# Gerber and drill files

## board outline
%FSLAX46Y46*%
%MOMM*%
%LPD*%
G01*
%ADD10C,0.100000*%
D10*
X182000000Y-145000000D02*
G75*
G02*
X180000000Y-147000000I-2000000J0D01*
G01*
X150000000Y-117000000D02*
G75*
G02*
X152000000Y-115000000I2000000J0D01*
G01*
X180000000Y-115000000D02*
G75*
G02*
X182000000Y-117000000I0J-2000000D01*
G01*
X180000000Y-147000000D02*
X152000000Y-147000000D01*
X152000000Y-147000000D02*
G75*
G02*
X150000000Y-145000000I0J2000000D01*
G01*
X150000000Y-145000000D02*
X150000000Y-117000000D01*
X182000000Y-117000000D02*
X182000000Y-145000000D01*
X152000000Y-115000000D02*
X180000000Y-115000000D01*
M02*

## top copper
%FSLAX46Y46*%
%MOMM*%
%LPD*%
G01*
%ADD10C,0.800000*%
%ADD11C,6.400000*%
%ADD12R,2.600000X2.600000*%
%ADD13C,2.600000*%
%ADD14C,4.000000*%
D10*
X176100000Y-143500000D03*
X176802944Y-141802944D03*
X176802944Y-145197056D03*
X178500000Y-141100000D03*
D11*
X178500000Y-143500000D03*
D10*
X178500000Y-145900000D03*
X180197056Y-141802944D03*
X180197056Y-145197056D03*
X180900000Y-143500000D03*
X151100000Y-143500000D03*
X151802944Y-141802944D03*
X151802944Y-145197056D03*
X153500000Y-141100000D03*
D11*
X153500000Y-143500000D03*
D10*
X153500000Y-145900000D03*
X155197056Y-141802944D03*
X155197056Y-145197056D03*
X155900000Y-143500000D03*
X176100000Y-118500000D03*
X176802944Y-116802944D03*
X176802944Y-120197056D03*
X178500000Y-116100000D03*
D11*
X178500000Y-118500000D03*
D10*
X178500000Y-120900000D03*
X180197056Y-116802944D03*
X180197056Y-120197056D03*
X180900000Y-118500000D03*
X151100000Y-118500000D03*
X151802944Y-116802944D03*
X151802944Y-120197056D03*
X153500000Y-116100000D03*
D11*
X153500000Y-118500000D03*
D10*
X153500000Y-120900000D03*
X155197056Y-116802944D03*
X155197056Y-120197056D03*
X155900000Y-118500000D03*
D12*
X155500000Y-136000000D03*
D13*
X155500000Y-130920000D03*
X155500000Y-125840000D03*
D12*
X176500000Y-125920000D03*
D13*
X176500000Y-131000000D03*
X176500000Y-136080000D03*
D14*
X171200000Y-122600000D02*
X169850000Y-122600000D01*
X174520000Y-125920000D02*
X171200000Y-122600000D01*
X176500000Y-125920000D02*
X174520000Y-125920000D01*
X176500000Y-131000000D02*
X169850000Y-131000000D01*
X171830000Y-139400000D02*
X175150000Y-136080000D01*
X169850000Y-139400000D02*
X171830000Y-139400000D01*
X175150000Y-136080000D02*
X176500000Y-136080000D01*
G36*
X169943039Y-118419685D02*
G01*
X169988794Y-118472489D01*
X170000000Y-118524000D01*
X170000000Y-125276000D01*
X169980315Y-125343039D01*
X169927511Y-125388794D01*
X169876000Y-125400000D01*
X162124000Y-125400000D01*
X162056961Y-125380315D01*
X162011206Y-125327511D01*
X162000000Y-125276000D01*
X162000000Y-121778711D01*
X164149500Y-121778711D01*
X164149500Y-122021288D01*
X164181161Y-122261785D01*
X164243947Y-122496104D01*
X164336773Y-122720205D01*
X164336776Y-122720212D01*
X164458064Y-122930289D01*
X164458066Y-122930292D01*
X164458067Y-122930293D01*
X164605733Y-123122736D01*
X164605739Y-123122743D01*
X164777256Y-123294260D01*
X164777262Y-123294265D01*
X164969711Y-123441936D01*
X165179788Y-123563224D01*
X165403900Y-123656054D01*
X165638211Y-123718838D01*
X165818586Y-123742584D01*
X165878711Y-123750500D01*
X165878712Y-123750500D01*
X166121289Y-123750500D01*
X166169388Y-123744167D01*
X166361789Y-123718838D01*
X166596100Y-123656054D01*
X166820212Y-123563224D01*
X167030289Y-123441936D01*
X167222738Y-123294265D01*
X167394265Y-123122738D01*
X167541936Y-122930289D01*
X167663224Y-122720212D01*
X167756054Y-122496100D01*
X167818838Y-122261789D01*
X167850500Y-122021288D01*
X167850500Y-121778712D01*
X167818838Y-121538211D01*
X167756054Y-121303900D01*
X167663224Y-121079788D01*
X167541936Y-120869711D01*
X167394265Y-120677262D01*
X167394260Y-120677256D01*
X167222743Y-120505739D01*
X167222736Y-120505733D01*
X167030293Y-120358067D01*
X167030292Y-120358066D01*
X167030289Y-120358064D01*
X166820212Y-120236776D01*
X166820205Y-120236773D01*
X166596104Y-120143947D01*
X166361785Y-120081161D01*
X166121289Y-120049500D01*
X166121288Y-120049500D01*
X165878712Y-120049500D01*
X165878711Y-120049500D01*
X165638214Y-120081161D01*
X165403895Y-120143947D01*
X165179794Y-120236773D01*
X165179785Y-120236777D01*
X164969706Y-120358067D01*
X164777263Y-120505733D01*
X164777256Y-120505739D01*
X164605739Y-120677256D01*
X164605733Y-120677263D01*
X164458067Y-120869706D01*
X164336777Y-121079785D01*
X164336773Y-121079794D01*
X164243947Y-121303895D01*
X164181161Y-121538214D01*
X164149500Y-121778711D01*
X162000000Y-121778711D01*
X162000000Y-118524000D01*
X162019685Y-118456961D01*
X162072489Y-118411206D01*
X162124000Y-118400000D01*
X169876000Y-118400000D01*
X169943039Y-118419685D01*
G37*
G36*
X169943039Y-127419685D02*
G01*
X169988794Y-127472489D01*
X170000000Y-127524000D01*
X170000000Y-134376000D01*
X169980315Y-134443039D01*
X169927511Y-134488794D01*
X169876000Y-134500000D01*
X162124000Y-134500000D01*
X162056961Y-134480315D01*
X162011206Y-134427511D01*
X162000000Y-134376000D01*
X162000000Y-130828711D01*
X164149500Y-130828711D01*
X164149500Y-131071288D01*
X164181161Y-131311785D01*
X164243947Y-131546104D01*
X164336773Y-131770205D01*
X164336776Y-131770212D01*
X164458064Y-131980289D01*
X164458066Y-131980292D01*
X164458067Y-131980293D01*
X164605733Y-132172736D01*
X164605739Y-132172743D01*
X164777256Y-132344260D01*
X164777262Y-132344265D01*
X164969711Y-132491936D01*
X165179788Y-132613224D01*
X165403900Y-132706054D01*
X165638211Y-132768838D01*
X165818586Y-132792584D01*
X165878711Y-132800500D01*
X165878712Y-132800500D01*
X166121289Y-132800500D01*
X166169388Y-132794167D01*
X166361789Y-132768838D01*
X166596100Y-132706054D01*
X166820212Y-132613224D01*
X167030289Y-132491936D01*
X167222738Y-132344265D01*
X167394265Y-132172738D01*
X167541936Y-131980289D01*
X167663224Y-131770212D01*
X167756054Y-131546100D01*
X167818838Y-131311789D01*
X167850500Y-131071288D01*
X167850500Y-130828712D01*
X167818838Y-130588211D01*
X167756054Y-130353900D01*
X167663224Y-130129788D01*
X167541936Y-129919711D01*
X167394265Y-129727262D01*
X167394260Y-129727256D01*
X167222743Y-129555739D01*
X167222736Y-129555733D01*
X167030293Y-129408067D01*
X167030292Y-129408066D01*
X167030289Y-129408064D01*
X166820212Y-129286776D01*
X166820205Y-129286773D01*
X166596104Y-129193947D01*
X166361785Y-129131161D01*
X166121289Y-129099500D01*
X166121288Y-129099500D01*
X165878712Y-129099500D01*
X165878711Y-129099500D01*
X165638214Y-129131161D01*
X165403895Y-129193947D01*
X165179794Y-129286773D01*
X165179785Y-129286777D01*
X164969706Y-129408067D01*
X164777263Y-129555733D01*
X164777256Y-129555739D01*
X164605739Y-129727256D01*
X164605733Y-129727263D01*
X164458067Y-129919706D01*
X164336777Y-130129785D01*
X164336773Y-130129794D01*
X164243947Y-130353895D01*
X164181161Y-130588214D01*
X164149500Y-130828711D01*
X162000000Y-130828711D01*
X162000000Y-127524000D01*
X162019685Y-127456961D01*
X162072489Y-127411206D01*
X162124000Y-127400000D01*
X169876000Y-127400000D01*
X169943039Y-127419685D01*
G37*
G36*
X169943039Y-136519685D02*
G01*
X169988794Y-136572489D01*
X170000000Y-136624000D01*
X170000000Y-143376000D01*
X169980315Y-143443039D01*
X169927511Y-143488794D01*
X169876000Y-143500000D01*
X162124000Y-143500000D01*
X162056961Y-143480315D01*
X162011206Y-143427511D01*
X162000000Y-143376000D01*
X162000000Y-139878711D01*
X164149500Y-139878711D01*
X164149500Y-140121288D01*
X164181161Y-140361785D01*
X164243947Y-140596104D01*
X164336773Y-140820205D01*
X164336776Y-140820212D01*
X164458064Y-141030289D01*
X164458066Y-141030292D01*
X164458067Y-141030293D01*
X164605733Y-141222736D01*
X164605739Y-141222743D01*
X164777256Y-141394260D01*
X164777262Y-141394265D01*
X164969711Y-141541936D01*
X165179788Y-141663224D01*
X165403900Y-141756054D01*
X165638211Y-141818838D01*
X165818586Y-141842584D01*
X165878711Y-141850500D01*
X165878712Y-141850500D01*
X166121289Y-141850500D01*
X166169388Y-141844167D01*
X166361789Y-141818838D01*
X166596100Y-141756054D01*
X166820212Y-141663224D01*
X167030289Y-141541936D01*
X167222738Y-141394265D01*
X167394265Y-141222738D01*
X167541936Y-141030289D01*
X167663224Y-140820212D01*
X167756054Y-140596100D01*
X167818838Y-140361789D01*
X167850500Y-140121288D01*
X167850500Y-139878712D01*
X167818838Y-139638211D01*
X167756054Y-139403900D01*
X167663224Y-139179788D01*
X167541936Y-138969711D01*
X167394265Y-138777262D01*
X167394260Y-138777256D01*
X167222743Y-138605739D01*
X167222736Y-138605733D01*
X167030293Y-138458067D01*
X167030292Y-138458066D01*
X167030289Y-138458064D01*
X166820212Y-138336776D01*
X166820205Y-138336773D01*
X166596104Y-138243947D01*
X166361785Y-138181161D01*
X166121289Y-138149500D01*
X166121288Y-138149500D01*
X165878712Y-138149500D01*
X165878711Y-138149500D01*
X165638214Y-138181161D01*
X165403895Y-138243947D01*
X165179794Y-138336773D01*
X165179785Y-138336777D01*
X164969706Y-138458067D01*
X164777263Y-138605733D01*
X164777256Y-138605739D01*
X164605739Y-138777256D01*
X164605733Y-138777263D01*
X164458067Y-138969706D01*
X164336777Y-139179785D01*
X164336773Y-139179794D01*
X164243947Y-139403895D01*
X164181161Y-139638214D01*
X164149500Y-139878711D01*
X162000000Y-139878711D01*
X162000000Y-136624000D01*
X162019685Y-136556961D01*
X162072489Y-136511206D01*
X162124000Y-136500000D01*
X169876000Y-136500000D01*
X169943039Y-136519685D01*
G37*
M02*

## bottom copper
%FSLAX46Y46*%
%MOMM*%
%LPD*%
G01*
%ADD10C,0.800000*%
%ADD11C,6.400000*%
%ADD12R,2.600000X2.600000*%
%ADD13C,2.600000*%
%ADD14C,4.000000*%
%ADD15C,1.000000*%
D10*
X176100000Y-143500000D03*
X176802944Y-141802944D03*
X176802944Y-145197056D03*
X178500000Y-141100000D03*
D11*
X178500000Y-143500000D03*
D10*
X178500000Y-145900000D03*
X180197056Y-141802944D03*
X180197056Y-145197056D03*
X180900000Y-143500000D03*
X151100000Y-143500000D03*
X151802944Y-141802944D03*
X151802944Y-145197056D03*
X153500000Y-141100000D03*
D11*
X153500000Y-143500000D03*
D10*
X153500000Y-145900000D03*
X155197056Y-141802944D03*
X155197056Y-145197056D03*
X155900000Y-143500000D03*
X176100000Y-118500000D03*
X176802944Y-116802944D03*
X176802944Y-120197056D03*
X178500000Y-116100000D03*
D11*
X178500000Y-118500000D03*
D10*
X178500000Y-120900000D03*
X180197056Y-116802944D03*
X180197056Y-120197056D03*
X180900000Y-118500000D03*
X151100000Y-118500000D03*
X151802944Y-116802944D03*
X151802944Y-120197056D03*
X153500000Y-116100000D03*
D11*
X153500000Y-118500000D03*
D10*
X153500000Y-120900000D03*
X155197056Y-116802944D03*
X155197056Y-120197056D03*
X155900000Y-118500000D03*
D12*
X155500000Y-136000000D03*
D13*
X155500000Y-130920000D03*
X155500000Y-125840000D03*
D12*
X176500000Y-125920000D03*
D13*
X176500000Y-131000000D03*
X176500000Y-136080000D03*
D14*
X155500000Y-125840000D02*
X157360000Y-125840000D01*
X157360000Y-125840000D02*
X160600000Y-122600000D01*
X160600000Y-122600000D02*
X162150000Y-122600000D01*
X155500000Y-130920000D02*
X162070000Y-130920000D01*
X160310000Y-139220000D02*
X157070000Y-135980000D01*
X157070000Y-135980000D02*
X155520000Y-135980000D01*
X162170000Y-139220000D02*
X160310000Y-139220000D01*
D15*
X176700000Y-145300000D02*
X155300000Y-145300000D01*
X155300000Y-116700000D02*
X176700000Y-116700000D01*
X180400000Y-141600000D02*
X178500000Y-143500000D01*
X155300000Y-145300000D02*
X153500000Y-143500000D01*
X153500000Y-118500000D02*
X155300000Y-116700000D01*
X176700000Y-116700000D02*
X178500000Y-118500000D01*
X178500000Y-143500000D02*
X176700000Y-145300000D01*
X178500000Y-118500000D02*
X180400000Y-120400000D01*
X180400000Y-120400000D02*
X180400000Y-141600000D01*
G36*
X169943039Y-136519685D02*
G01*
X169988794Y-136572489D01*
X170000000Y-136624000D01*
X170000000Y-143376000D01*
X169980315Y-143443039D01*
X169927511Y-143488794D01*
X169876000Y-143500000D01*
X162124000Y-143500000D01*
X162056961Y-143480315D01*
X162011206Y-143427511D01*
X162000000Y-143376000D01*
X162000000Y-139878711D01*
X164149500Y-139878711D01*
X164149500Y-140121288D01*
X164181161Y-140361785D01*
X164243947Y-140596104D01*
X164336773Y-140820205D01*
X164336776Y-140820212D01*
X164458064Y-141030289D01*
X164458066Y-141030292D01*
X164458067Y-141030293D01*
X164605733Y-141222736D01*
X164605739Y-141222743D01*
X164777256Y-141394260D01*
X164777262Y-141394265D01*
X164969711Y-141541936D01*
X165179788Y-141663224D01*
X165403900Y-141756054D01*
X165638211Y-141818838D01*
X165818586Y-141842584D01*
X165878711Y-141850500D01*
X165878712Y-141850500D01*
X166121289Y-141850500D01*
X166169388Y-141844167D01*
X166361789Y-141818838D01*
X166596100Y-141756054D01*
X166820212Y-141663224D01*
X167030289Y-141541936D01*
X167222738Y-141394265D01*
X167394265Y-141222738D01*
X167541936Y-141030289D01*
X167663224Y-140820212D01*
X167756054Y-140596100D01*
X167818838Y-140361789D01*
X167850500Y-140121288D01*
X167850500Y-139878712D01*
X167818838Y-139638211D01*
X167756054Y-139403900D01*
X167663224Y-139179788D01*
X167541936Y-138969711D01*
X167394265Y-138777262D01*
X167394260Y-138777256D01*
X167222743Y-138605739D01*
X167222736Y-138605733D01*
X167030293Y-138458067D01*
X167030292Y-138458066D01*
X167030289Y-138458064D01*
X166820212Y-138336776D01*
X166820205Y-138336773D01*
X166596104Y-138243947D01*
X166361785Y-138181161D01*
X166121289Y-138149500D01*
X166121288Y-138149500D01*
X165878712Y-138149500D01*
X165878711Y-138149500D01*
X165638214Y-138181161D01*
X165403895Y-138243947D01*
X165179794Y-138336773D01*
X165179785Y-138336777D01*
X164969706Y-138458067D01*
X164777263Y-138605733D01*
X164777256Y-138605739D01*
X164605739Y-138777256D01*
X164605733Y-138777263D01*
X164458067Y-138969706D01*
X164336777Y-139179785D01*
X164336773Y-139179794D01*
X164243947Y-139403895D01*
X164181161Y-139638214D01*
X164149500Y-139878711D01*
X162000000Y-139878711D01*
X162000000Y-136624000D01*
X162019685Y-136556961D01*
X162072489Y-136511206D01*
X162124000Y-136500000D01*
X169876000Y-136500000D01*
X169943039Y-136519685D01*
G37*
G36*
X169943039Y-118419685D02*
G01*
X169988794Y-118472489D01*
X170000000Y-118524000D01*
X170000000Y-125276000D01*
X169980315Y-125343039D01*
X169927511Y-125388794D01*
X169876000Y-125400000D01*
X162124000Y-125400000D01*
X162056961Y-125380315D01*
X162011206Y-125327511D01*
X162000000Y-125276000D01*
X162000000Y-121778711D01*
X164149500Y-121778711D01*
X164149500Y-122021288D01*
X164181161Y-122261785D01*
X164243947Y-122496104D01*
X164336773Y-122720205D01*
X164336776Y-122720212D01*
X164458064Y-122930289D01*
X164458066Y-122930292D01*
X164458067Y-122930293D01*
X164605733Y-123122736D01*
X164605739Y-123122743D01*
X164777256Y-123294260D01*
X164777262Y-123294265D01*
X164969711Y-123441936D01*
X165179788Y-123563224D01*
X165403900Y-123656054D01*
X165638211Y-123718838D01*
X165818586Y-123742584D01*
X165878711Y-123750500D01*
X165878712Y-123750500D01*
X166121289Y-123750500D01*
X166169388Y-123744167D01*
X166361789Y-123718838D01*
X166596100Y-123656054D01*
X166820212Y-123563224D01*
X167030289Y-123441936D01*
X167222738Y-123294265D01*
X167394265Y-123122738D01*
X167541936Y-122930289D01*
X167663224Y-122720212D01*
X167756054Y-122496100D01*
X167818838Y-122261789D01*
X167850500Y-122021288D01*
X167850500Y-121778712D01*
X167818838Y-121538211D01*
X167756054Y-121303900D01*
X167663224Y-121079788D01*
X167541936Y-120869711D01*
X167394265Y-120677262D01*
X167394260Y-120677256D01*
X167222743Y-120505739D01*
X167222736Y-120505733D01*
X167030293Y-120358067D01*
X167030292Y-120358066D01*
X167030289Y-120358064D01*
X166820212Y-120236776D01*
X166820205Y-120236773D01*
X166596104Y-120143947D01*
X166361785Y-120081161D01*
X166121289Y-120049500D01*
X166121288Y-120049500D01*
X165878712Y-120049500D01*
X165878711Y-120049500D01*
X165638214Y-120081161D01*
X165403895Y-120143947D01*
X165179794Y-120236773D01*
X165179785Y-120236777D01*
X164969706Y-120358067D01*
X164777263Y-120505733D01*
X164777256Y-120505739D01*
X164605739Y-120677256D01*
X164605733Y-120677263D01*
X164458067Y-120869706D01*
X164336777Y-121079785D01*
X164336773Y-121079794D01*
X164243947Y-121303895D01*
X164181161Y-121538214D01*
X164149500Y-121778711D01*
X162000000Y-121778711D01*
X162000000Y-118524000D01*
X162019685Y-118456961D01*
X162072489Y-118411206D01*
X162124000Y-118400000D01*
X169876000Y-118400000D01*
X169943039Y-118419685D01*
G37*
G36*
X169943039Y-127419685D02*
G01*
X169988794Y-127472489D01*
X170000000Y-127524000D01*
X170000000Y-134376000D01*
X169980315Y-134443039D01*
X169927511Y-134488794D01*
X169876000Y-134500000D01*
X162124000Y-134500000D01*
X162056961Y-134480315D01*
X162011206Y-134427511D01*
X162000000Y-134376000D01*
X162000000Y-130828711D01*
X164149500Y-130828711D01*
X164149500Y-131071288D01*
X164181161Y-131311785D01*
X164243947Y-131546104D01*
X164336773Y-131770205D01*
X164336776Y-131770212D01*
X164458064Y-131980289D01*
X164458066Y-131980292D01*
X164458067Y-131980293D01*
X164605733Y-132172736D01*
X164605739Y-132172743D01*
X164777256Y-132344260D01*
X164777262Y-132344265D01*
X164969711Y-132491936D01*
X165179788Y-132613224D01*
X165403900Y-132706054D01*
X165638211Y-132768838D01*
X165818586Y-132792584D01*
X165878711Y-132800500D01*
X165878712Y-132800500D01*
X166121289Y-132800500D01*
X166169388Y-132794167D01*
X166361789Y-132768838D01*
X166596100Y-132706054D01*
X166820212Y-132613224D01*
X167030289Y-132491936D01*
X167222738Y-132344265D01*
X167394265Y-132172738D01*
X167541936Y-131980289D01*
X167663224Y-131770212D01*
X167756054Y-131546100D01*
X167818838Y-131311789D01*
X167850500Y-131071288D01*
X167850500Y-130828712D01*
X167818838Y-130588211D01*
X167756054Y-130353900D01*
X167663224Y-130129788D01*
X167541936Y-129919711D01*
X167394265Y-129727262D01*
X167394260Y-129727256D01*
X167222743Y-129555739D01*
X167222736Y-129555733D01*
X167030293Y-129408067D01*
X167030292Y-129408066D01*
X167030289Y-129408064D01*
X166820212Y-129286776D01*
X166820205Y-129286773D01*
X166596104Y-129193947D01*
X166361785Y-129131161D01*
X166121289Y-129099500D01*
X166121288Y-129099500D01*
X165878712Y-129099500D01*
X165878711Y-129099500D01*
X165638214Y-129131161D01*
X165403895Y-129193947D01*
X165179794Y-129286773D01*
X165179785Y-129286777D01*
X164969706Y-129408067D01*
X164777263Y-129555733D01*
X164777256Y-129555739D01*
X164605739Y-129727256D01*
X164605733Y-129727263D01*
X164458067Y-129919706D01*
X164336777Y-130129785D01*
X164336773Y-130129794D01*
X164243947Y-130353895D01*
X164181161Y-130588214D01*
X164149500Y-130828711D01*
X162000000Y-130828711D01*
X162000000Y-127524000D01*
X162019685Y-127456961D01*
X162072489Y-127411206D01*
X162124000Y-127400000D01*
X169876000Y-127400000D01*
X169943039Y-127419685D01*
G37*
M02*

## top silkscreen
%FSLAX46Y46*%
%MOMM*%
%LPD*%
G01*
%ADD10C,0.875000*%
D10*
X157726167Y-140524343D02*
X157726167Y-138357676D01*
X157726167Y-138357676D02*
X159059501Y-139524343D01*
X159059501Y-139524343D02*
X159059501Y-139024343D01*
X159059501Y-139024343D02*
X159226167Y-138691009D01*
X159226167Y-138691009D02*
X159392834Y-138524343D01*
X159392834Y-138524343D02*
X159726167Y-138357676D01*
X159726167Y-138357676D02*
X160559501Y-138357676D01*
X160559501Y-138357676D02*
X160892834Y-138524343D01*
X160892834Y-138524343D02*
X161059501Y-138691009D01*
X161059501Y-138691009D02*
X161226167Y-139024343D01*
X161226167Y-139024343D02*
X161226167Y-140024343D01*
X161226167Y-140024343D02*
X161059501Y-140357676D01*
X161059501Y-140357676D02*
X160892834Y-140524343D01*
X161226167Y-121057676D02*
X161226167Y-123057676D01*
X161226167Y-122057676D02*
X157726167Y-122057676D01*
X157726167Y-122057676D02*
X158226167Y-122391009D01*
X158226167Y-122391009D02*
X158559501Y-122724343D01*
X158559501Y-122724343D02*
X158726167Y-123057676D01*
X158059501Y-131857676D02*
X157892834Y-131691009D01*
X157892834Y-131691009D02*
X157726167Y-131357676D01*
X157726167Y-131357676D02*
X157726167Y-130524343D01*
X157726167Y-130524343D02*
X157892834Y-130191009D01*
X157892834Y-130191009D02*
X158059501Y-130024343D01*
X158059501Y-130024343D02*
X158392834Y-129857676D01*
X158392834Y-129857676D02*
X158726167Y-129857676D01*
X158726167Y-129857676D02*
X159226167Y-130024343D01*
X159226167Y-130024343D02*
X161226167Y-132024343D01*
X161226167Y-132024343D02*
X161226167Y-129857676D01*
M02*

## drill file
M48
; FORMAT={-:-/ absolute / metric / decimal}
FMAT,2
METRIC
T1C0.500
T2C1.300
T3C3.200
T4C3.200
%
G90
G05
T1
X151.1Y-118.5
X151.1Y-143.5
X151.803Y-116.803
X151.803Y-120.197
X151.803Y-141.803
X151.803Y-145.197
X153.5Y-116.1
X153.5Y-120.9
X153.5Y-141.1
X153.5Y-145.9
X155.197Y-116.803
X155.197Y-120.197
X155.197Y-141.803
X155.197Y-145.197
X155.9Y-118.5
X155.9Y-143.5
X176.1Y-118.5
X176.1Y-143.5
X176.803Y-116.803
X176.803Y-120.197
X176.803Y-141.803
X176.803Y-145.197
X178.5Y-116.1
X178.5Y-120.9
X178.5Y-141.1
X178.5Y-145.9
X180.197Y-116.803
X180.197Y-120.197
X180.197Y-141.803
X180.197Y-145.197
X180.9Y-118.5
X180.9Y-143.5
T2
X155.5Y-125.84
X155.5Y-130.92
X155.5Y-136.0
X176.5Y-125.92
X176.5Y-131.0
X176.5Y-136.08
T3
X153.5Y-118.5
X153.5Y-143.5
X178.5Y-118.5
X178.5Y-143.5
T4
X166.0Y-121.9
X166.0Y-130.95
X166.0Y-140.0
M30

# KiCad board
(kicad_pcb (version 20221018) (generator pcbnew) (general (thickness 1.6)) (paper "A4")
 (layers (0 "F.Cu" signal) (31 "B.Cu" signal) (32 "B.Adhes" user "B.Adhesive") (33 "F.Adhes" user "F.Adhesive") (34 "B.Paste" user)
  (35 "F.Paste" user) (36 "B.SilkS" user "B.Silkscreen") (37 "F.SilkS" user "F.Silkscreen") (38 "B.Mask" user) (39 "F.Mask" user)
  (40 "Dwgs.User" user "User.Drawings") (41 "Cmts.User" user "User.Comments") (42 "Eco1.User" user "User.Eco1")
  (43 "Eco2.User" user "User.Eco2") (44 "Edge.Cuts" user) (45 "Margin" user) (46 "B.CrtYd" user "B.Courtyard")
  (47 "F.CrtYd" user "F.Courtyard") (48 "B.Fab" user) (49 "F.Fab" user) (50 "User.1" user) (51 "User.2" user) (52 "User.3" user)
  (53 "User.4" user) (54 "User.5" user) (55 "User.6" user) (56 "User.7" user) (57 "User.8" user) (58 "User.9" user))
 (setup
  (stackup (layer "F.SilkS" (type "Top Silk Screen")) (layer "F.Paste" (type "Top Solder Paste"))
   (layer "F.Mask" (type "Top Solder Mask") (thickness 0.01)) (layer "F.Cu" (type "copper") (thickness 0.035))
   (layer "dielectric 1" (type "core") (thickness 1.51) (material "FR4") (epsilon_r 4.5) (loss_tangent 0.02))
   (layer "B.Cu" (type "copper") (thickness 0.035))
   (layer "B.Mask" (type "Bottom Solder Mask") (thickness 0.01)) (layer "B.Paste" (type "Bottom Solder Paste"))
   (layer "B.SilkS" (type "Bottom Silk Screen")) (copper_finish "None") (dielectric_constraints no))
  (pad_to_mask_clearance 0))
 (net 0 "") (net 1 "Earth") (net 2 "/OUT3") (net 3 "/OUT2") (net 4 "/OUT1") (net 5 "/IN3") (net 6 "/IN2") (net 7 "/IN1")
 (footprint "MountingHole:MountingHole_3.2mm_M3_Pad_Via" (layer "F.Cu") (at 178.5 143.5)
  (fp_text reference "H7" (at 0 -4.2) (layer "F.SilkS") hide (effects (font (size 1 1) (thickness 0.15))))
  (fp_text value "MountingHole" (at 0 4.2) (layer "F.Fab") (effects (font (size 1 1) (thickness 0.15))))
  (pad "1" thru_hole circle (at -2.4 0) (size 0.8 0.8) (drill 0.5) (layers "*.Cu" "*.Mask") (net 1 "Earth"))
  (pad "1" thru_hole circle (at -1.697056 -1.697056) (size 0.8 0.8) (drill 0.5) (layers "*.Cu" "*.Mask") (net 1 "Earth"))
  (pad "1" thru_hole circle (at -1.697056 1.697056) (size 0.8 0.8) (drill 0.5) (layers "*.Cu" "*.Mask") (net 1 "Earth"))
  (pad "1" thru_hole circle (at 0 -2.4) (size 0.8 0.8) (drill 0.5) (layers "*.Cu" "*.Mask") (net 1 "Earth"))
  (pad "1" thru_hole circle (at 0 0) (size 6.4 6.4) (drill 3.2) (layers "*.Cu" "*.Mask") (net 1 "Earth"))
  (pad "1" thru_hole circle (at 0 2.4) (size 0.8 0.8) (drill 0.5) (layers "*.Cu" "*.Mask") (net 1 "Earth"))
  (pad "1" thru_hole circle (at 1.697056 -1.697056) (size 0.8 0.8) (drill 0.5) (layers "*.Cu" "*.Mask") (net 1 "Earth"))
  (pad "1" thru_hole circle (at 1.697056 1.697056) (size 0.8 0.8) (drill 0.5) (layers "*.Cu" "*.Mask") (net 1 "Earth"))
  (pad "1" thru_hole circle (at 2.4 0) (size 0.8 0.8) (drill 0.5) (layers "*.Cu" "*.Mask") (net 1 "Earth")))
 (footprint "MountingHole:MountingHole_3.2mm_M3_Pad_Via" (layer "F.Cu") (at 153.5 143.5)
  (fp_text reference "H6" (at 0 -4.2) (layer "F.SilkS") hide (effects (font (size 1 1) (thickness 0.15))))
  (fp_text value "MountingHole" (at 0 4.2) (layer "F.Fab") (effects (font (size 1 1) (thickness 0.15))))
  (pad "1" thru_hole circle (at -2.4 0) (size 0.8 0.8) (drill 0.5) (layers "*.Cu" "*.Mask") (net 1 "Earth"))
  (pad "1" thru_hole circle (at -1.697056 -1.697056) (size 0.8 0.8) (drill 0.5) (layers "*.Cu" "*.Mask") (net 1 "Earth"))
  (pad "1" thru_hole circle (at -1.697056 1.697056) (size 0.8 0.8) (drill 0.5) (layers "*.Cu" "*.Mask") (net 1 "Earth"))
  (pad "1" thru_hole circle (at 0 -2.4) (size 0.8 0.8) (drill 0.5) (layers "*.Cu" "*.Mask") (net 1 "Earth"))
  (pad "1" thru_hole circle (at 0 0) (size 6.4 6.4) (drill 3.2) (layers "*.Cu" "*.Mask") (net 1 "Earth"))
  (pad "1" thru_hole circle (at 0 2.4) (size 0.8 0.8) (drill 0.5) (layers "*.Cu" "*.Mask") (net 1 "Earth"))
  (pad "1" thru_hole circle (at 1.697056 -1.697056) (size 0.8 0.8) (drill 0.5) (layers "*.Cu" "*.Mask") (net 1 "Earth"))
  (pad "1" thru_hole circle (at 1.697056 1.697056) (size 0.8 0.8) (drill 0.5) (layers "*.Cu" "*.Mask") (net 1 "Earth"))
  (pad "1" thru_hole circle (at 2.4 0) (size 0.8 0.8) (drill 0.5) (layers "*.Cu" "*.Mask") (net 1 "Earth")))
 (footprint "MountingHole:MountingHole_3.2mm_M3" (layer "F.Cu") (at 166 130.95)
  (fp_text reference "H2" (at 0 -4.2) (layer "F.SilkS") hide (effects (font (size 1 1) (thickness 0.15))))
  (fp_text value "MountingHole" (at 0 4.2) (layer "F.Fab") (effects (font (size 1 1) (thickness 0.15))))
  (pad "" np_thru_hole circle (at 0 0) (size 3.2 3.2) (drill 3.2) (layers "*.Cu" "*.Mask")))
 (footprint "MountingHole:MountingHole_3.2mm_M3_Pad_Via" (layer "F.Cu") (at 178.5 118.5)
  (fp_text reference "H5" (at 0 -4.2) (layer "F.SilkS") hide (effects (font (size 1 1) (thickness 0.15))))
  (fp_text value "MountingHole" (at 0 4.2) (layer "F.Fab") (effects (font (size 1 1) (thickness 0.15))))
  (pad "1" thru_hole circle (at -2.4 0) (size 0.8 0.8) (drill 0.5) (layers "*.Cu" "*.Mask") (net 1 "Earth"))
  (pad "1" thru_hole circle (at -1.697056 -1.697056) (size 0.8 0.8) (drill 0.5) (layers "*.Cu" "*.Mask") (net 1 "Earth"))
  (pad "1" thru_hole circle (at -1.697056 1.697056) (size 0.8 0.8) (drill 0.5) (layers "*.Cu" "*.Mask") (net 1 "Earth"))
  (pad "1" thru_hole circle (at 0 -2.4) (size 0.8 0.8) (drill 0.5) (layers "*.Cu" "*.Mask") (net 1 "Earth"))
  (pad "1" thru_hole circle (at 0 0) (size 6.4 6.4) (drill 3.2) (layers "*.Cu" "*.Mask") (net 1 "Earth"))
  (pad "1" thru_hole circle (at 0 2.4) (size 0.8 0.8) (drill 0.5) (layers "*.Cu" "*.Mask") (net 1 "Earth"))
  (pad "1" thru_hole circle (at 1.697056 -1.697056) (size 0.8 0.8) (drill 0.5) (layers "*.Cu" "*.Mask") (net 1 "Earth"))
  (pad "1" thru_hole circle (at 1.697056 1.697056) (size 0.8 0.8) (drill 0.5) (layers "*.Cu" "*.Mask") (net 1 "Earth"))
  (pad "1" thru_hole circle (at 2.4 0) (size 0.8 0.8) (drill 0.5) (layers "*.Cu" "*.Mask") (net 1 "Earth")))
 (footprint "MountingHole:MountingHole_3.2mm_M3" (layer "F.Cu") (at 166 121.9)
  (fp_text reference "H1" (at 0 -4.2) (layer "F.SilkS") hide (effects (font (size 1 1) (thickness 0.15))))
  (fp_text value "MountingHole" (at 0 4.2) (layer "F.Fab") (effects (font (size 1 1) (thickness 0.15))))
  (pad "" np_thru_hole circle (at 0 0) (size 3.2 3.2) (drill 3.2) (layers "*.Cu" "*.Mask")))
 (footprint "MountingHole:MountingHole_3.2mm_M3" (layer "F.Cu") (at 166 140)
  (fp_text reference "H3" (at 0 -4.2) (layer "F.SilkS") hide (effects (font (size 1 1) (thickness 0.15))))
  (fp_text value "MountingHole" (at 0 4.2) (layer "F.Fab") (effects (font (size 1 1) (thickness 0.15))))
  (pad "" np_thru_hole circle (at 0 0) (size 3.2 3.2) (drill 3.2) (layers "*.Cu" "*.Mask")))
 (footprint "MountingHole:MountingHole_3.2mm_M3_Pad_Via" (layer "F.Cu") (at 153.5 118.5)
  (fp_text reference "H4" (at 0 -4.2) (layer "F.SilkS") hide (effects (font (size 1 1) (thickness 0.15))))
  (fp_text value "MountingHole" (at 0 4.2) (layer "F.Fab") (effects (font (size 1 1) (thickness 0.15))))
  (pad "1" thru_hole circle (at -2.4 0) (size 0.8 0.8) (drill 0.5) (layers "*.Cu" "*.Mask") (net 1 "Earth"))
  (pad "1" thru_hole circle (at -1.697056 -1.697056) (size 0.8 0.8) (drill 0.5) (layers "*.Cu" "*.Mask") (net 1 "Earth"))
  (pad "1" thru_hole circle (at -1.697056 1.697056) (size 0.8 0.8) (drill 0.5) (layers "*.Cu" "*.Mask") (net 1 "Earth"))
  (pad "1" thru_hole circle (at 0 -2.4) (size 0.8 0.8) (drill 0.5) (layers "*.Cu" "*.Mask") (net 1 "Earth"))
  (pad "1" thru_hole circle (at 0 0) (size 6.4 6.4) (drill 3.2) (layers "*.Cu" "*.Mask") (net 1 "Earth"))
  (pad "1" thru_hole circle (at 0 2.4) (size 0.8 0.8) (drill 0.5) (layers "*.Cu" "*.Mask") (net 1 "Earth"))
  (pad "1" thru_hole circle (at 1.697056 -1.697056) (size 0.8 0.8) (drill 0.5) (layers "*.Cu" "*.Mask") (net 1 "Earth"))
  (pad "1" thru_hole circle (at 1.697056 1.697056) (size 0.8 0.8) (drill 0.5) (layers "*.Cu" "*.Mask") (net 1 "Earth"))
  (pad "1" thru_hole circle (at 2.4 0) (size 0.8 0.8) (drill 0.5) (layers "*.Cu" "*.Mask") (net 1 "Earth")))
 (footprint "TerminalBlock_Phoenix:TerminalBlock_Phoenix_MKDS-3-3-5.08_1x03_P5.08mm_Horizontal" (layer "B.Cu") (at 155.5 136 90)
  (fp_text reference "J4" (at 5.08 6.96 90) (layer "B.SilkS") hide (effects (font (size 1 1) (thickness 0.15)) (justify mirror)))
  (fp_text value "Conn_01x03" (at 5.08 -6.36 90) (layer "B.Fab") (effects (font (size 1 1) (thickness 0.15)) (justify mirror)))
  (pad "1" thru_hole rect (at 0 0 90) (size 2.6 2.6) (drill 1.3) (layers "*.Cu" "*.Mask") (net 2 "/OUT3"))
  (pad "2" thru_hole circle (at 5.08 0 90) (size 2.6 2.6) (drill 1.3) (layers "*.Cu" "*.Mask") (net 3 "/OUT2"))
  (pad "3" thru_hole circle (at 10.16 0 90) (size 2.6 2.6) (drill 1.3) (layers "*.Cu" "*.Mask") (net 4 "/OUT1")))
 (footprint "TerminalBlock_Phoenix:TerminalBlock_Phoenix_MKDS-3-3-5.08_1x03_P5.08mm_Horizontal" (layer "B.Cu") (at 176.5 125.92 -90)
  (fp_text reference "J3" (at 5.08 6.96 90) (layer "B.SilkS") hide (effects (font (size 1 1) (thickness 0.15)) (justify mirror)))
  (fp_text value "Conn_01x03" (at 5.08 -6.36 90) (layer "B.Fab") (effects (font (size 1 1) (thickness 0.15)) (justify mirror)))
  (pad "1" thru_hole rect (at 0 0 270) (size 2.6 2.6) (drill 1.3) (layers "*.Cu" "*.Mask") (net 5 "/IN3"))
  (pad "2" thru_hole circle (at 5.08 0 270) (size 2.6 2.6) (drill 1.3) (layers "*.Cu" "*.Mask") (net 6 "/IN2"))
  (pad "3" thru_hole circle (at 10.16 0 270) (size 2.6 2.6) (drill 1.3) (layers "*.Cu" "*.Mask") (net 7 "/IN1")))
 (gr_arc (start 182 145) (mid 181.414214 146.414214) (end 180 147) (stroke (width 0.1) (type default)) (layer "Edge.Cuts"))
 (gr_arc (start 150 117) (mid 150.585786 115.585786) (end 152 115) (stroke (width 0.1) (type default)) (layer "Edge.Cuts"))
 (gr_arc (start 180 115) (mid 181.414214 115.585786) (end 182 117) (stroke (width 0.1) (type default)) (layer "Edge.Cuts"))
 (gr_line (start 180 147) (end 152 147) (stroke (width 0.1) (type default)) (layer "Edge.Cuts"))
 (gr_arc (start 152 147) (mid 150.585786 146.414214) (end 150 145) (stroke (width 0.1) (type default)) (layer "Edge.Cuts"))
 (gr_line (start 150 145) (end 150 117) (stroke (width 0.1) (type default)) (layer "Edge.Cuts"))
 (gr_line (start 182 117) (end 182 145) (stroke (width 0.1) (type default)) (layer "Edge.Cuts"))
 (gr_line (start 152 115) (end 180 115) (stroke (width 0.1) (type default)) (layer "Edge.Cuts"))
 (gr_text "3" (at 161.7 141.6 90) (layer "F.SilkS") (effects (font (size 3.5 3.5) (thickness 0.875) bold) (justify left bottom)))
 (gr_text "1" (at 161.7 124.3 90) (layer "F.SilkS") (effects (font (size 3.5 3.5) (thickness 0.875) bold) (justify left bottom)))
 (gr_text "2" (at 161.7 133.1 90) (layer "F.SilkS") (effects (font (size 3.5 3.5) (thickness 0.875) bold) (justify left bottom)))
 (segment (start 155.5 125.84) (end 157.36 125.84) (width 4) (layer "B.Cu") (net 4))
 (segment (start 157.36 125.84) (end 160.6 122.6) (width 4) (layer "B.Cu") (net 4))
 (segment (start 160.6 122.6) (end 162.15 122.6) (width 4) (layer "B.Cu") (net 4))
 (segment (start 155.5 130.92) (end 162.07 130.92) (width 4) (layer "B.Cu") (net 3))
 (segment (start 160.31 139.22) (end 157.07 135.98) (width 4) (layer "B.Cu") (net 2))
 (segment (start 157.07 135.98) (end 155.52 135.98) (width 4) (layer "B.Cu") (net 2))
 (segment (start 162.17 139.22) (end 160.31 139.22) (width 4) (layer "B.Cu") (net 2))
 (segment (start 171.2 122.6) (end 169.85 122.6) (width 4) (layer "F.Cu") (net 5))
 (segment (start 174.52 125.92) (end 171.2 122.6) (width 4) (layer "F.Cu") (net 5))
 (segment (start 176.5 125.92) (end 174.52 125.92) (width 4) (layer "F.Cu") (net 5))
 (segment (start 176.5 131) (end 169.85 131) (width 4) (layer "F.Cu") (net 6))
 (segment (start 171.83 139.4) (end 175.15 136.08) (width 4) (layer "F.Cu") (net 7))
 (segment (start 169.85 139.4) (end 171.83 139.4) (width 4) (layer "F.Cu") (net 7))
 (segment (start 175.15 136.08) (end 176.5 136.08) (width 4) (layer "F.Cu") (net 7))
 (segment (start 176.7 145.3) (end 155.3 145.3) (width 1) (layer "B.Cu") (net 1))
 (segment (start 155.3 116.7) (end 176.7 116.7) (width 1) (layer "B.Cu") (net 1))
 (segment (start 180.4 141.6) (end 178.5 143.5) (width 1) (layer "B.Cu") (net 1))
 (segment (start 155.3 145.3) (end 153.5 143.5) (width 1) (layer "B.Cu") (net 1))
 (segment (start 153.5 118.5) (end 155.3 116.7) (width 1) (layer "B.Cu") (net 1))
 (segment (start 176.7 116.7) (end 178.5 118.5) (width 1) (layer "B.Cu") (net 1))
 (segment (start 178.5 143.5) (end 176.7 145.3) (width 1) (layer "B.Cu") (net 1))
 (segment (start 178.5 118.5) (end 180.4 120.4) (width 1) (layer "B.Cu") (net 1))
 (segment (start 180.4 120.4) (end 180.4 141.6) (width 1) (layer "B.Cu") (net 1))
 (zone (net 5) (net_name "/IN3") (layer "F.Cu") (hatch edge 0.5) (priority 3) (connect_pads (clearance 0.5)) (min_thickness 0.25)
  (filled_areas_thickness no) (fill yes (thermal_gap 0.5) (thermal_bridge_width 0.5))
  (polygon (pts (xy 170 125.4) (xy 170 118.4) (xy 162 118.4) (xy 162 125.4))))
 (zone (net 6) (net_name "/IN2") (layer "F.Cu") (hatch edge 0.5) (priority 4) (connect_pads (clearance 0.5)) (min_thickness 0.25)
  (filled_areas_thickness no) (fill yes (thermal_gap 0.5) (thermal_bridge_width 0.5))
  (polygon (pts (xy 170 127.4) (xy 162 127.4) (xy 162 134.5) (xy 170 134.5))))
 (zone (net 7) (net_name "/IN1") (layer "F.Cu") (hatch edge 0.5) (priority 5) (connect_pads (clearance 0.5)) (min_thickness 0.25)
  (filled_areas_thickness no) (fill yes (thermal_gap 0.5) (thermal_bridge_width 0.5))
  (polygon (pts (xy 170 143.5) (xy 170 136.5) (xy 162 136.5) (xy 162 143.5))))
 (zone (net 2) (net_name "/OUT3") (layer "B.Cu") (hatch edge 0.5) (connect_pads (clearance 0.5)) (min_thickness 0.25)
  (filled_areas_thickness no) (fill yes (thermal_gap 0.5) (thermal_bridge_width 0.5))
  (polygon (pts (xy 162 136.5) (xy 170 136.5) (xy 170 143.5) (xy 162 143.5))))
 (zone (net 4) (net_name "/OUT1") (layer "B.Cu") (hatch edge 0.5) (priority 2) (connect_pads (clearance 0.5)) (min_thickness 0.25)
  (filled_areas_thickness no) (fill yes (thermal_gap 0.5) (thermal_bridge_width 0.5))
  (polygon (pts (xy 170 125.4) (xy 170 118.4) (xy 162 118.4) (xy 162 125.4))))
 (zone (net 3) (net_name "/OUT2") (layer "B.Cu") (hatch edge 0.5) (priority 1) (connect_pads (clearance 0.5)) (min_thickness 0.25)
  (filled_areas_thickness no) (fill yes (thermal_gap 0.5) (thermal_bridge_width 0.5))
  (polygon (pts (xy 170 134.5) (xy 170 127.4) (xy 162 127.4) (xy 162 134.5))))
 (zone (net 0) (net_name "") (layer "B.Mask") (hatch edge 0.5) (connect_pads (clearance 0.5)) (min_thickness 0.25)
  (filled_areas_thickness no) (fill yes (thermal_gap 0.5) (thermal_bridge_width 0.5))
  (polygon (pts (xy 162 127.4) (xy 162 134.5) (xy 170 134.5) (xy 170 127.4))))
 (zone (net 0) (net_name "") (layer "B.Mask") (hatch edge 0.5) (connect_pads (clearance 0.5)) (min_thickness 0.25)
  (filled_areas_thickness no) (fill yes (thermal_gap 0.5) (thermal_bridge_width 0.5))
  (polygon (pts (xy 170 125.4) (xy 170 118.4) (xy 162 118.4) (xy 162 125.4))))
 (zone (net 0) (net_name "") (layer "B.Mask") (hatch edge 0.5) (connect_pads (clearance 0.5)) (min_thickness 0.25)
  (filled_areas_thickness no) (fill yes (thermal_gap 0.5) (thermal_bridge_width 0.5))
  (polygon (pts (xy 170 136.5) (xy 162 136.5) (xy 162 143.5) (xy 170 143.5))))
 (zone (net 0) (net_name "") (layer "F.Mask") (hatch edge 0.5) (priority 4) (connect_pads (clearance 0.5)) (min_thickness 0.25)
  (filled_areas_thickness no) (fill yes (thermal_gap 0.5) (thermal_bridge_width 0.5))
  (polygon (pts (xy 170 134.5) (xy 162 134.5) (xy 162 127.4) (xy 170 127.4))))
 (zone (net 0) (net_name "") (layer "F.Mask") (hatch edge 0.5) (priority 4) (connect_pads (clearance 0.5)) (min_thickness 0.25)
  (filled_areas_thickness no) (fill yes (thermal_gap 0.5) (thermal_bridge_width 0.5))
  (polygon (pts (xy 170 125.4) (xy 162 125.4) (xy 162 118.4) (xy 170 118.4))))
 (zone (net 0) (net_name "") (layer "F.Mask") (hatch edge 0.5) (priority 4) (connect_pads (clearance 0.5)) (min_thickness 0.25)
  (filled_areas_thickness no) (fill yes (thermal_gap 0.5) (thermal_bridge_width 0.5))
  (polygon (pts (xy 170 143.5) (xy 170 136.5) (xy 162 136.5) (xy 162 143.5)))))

